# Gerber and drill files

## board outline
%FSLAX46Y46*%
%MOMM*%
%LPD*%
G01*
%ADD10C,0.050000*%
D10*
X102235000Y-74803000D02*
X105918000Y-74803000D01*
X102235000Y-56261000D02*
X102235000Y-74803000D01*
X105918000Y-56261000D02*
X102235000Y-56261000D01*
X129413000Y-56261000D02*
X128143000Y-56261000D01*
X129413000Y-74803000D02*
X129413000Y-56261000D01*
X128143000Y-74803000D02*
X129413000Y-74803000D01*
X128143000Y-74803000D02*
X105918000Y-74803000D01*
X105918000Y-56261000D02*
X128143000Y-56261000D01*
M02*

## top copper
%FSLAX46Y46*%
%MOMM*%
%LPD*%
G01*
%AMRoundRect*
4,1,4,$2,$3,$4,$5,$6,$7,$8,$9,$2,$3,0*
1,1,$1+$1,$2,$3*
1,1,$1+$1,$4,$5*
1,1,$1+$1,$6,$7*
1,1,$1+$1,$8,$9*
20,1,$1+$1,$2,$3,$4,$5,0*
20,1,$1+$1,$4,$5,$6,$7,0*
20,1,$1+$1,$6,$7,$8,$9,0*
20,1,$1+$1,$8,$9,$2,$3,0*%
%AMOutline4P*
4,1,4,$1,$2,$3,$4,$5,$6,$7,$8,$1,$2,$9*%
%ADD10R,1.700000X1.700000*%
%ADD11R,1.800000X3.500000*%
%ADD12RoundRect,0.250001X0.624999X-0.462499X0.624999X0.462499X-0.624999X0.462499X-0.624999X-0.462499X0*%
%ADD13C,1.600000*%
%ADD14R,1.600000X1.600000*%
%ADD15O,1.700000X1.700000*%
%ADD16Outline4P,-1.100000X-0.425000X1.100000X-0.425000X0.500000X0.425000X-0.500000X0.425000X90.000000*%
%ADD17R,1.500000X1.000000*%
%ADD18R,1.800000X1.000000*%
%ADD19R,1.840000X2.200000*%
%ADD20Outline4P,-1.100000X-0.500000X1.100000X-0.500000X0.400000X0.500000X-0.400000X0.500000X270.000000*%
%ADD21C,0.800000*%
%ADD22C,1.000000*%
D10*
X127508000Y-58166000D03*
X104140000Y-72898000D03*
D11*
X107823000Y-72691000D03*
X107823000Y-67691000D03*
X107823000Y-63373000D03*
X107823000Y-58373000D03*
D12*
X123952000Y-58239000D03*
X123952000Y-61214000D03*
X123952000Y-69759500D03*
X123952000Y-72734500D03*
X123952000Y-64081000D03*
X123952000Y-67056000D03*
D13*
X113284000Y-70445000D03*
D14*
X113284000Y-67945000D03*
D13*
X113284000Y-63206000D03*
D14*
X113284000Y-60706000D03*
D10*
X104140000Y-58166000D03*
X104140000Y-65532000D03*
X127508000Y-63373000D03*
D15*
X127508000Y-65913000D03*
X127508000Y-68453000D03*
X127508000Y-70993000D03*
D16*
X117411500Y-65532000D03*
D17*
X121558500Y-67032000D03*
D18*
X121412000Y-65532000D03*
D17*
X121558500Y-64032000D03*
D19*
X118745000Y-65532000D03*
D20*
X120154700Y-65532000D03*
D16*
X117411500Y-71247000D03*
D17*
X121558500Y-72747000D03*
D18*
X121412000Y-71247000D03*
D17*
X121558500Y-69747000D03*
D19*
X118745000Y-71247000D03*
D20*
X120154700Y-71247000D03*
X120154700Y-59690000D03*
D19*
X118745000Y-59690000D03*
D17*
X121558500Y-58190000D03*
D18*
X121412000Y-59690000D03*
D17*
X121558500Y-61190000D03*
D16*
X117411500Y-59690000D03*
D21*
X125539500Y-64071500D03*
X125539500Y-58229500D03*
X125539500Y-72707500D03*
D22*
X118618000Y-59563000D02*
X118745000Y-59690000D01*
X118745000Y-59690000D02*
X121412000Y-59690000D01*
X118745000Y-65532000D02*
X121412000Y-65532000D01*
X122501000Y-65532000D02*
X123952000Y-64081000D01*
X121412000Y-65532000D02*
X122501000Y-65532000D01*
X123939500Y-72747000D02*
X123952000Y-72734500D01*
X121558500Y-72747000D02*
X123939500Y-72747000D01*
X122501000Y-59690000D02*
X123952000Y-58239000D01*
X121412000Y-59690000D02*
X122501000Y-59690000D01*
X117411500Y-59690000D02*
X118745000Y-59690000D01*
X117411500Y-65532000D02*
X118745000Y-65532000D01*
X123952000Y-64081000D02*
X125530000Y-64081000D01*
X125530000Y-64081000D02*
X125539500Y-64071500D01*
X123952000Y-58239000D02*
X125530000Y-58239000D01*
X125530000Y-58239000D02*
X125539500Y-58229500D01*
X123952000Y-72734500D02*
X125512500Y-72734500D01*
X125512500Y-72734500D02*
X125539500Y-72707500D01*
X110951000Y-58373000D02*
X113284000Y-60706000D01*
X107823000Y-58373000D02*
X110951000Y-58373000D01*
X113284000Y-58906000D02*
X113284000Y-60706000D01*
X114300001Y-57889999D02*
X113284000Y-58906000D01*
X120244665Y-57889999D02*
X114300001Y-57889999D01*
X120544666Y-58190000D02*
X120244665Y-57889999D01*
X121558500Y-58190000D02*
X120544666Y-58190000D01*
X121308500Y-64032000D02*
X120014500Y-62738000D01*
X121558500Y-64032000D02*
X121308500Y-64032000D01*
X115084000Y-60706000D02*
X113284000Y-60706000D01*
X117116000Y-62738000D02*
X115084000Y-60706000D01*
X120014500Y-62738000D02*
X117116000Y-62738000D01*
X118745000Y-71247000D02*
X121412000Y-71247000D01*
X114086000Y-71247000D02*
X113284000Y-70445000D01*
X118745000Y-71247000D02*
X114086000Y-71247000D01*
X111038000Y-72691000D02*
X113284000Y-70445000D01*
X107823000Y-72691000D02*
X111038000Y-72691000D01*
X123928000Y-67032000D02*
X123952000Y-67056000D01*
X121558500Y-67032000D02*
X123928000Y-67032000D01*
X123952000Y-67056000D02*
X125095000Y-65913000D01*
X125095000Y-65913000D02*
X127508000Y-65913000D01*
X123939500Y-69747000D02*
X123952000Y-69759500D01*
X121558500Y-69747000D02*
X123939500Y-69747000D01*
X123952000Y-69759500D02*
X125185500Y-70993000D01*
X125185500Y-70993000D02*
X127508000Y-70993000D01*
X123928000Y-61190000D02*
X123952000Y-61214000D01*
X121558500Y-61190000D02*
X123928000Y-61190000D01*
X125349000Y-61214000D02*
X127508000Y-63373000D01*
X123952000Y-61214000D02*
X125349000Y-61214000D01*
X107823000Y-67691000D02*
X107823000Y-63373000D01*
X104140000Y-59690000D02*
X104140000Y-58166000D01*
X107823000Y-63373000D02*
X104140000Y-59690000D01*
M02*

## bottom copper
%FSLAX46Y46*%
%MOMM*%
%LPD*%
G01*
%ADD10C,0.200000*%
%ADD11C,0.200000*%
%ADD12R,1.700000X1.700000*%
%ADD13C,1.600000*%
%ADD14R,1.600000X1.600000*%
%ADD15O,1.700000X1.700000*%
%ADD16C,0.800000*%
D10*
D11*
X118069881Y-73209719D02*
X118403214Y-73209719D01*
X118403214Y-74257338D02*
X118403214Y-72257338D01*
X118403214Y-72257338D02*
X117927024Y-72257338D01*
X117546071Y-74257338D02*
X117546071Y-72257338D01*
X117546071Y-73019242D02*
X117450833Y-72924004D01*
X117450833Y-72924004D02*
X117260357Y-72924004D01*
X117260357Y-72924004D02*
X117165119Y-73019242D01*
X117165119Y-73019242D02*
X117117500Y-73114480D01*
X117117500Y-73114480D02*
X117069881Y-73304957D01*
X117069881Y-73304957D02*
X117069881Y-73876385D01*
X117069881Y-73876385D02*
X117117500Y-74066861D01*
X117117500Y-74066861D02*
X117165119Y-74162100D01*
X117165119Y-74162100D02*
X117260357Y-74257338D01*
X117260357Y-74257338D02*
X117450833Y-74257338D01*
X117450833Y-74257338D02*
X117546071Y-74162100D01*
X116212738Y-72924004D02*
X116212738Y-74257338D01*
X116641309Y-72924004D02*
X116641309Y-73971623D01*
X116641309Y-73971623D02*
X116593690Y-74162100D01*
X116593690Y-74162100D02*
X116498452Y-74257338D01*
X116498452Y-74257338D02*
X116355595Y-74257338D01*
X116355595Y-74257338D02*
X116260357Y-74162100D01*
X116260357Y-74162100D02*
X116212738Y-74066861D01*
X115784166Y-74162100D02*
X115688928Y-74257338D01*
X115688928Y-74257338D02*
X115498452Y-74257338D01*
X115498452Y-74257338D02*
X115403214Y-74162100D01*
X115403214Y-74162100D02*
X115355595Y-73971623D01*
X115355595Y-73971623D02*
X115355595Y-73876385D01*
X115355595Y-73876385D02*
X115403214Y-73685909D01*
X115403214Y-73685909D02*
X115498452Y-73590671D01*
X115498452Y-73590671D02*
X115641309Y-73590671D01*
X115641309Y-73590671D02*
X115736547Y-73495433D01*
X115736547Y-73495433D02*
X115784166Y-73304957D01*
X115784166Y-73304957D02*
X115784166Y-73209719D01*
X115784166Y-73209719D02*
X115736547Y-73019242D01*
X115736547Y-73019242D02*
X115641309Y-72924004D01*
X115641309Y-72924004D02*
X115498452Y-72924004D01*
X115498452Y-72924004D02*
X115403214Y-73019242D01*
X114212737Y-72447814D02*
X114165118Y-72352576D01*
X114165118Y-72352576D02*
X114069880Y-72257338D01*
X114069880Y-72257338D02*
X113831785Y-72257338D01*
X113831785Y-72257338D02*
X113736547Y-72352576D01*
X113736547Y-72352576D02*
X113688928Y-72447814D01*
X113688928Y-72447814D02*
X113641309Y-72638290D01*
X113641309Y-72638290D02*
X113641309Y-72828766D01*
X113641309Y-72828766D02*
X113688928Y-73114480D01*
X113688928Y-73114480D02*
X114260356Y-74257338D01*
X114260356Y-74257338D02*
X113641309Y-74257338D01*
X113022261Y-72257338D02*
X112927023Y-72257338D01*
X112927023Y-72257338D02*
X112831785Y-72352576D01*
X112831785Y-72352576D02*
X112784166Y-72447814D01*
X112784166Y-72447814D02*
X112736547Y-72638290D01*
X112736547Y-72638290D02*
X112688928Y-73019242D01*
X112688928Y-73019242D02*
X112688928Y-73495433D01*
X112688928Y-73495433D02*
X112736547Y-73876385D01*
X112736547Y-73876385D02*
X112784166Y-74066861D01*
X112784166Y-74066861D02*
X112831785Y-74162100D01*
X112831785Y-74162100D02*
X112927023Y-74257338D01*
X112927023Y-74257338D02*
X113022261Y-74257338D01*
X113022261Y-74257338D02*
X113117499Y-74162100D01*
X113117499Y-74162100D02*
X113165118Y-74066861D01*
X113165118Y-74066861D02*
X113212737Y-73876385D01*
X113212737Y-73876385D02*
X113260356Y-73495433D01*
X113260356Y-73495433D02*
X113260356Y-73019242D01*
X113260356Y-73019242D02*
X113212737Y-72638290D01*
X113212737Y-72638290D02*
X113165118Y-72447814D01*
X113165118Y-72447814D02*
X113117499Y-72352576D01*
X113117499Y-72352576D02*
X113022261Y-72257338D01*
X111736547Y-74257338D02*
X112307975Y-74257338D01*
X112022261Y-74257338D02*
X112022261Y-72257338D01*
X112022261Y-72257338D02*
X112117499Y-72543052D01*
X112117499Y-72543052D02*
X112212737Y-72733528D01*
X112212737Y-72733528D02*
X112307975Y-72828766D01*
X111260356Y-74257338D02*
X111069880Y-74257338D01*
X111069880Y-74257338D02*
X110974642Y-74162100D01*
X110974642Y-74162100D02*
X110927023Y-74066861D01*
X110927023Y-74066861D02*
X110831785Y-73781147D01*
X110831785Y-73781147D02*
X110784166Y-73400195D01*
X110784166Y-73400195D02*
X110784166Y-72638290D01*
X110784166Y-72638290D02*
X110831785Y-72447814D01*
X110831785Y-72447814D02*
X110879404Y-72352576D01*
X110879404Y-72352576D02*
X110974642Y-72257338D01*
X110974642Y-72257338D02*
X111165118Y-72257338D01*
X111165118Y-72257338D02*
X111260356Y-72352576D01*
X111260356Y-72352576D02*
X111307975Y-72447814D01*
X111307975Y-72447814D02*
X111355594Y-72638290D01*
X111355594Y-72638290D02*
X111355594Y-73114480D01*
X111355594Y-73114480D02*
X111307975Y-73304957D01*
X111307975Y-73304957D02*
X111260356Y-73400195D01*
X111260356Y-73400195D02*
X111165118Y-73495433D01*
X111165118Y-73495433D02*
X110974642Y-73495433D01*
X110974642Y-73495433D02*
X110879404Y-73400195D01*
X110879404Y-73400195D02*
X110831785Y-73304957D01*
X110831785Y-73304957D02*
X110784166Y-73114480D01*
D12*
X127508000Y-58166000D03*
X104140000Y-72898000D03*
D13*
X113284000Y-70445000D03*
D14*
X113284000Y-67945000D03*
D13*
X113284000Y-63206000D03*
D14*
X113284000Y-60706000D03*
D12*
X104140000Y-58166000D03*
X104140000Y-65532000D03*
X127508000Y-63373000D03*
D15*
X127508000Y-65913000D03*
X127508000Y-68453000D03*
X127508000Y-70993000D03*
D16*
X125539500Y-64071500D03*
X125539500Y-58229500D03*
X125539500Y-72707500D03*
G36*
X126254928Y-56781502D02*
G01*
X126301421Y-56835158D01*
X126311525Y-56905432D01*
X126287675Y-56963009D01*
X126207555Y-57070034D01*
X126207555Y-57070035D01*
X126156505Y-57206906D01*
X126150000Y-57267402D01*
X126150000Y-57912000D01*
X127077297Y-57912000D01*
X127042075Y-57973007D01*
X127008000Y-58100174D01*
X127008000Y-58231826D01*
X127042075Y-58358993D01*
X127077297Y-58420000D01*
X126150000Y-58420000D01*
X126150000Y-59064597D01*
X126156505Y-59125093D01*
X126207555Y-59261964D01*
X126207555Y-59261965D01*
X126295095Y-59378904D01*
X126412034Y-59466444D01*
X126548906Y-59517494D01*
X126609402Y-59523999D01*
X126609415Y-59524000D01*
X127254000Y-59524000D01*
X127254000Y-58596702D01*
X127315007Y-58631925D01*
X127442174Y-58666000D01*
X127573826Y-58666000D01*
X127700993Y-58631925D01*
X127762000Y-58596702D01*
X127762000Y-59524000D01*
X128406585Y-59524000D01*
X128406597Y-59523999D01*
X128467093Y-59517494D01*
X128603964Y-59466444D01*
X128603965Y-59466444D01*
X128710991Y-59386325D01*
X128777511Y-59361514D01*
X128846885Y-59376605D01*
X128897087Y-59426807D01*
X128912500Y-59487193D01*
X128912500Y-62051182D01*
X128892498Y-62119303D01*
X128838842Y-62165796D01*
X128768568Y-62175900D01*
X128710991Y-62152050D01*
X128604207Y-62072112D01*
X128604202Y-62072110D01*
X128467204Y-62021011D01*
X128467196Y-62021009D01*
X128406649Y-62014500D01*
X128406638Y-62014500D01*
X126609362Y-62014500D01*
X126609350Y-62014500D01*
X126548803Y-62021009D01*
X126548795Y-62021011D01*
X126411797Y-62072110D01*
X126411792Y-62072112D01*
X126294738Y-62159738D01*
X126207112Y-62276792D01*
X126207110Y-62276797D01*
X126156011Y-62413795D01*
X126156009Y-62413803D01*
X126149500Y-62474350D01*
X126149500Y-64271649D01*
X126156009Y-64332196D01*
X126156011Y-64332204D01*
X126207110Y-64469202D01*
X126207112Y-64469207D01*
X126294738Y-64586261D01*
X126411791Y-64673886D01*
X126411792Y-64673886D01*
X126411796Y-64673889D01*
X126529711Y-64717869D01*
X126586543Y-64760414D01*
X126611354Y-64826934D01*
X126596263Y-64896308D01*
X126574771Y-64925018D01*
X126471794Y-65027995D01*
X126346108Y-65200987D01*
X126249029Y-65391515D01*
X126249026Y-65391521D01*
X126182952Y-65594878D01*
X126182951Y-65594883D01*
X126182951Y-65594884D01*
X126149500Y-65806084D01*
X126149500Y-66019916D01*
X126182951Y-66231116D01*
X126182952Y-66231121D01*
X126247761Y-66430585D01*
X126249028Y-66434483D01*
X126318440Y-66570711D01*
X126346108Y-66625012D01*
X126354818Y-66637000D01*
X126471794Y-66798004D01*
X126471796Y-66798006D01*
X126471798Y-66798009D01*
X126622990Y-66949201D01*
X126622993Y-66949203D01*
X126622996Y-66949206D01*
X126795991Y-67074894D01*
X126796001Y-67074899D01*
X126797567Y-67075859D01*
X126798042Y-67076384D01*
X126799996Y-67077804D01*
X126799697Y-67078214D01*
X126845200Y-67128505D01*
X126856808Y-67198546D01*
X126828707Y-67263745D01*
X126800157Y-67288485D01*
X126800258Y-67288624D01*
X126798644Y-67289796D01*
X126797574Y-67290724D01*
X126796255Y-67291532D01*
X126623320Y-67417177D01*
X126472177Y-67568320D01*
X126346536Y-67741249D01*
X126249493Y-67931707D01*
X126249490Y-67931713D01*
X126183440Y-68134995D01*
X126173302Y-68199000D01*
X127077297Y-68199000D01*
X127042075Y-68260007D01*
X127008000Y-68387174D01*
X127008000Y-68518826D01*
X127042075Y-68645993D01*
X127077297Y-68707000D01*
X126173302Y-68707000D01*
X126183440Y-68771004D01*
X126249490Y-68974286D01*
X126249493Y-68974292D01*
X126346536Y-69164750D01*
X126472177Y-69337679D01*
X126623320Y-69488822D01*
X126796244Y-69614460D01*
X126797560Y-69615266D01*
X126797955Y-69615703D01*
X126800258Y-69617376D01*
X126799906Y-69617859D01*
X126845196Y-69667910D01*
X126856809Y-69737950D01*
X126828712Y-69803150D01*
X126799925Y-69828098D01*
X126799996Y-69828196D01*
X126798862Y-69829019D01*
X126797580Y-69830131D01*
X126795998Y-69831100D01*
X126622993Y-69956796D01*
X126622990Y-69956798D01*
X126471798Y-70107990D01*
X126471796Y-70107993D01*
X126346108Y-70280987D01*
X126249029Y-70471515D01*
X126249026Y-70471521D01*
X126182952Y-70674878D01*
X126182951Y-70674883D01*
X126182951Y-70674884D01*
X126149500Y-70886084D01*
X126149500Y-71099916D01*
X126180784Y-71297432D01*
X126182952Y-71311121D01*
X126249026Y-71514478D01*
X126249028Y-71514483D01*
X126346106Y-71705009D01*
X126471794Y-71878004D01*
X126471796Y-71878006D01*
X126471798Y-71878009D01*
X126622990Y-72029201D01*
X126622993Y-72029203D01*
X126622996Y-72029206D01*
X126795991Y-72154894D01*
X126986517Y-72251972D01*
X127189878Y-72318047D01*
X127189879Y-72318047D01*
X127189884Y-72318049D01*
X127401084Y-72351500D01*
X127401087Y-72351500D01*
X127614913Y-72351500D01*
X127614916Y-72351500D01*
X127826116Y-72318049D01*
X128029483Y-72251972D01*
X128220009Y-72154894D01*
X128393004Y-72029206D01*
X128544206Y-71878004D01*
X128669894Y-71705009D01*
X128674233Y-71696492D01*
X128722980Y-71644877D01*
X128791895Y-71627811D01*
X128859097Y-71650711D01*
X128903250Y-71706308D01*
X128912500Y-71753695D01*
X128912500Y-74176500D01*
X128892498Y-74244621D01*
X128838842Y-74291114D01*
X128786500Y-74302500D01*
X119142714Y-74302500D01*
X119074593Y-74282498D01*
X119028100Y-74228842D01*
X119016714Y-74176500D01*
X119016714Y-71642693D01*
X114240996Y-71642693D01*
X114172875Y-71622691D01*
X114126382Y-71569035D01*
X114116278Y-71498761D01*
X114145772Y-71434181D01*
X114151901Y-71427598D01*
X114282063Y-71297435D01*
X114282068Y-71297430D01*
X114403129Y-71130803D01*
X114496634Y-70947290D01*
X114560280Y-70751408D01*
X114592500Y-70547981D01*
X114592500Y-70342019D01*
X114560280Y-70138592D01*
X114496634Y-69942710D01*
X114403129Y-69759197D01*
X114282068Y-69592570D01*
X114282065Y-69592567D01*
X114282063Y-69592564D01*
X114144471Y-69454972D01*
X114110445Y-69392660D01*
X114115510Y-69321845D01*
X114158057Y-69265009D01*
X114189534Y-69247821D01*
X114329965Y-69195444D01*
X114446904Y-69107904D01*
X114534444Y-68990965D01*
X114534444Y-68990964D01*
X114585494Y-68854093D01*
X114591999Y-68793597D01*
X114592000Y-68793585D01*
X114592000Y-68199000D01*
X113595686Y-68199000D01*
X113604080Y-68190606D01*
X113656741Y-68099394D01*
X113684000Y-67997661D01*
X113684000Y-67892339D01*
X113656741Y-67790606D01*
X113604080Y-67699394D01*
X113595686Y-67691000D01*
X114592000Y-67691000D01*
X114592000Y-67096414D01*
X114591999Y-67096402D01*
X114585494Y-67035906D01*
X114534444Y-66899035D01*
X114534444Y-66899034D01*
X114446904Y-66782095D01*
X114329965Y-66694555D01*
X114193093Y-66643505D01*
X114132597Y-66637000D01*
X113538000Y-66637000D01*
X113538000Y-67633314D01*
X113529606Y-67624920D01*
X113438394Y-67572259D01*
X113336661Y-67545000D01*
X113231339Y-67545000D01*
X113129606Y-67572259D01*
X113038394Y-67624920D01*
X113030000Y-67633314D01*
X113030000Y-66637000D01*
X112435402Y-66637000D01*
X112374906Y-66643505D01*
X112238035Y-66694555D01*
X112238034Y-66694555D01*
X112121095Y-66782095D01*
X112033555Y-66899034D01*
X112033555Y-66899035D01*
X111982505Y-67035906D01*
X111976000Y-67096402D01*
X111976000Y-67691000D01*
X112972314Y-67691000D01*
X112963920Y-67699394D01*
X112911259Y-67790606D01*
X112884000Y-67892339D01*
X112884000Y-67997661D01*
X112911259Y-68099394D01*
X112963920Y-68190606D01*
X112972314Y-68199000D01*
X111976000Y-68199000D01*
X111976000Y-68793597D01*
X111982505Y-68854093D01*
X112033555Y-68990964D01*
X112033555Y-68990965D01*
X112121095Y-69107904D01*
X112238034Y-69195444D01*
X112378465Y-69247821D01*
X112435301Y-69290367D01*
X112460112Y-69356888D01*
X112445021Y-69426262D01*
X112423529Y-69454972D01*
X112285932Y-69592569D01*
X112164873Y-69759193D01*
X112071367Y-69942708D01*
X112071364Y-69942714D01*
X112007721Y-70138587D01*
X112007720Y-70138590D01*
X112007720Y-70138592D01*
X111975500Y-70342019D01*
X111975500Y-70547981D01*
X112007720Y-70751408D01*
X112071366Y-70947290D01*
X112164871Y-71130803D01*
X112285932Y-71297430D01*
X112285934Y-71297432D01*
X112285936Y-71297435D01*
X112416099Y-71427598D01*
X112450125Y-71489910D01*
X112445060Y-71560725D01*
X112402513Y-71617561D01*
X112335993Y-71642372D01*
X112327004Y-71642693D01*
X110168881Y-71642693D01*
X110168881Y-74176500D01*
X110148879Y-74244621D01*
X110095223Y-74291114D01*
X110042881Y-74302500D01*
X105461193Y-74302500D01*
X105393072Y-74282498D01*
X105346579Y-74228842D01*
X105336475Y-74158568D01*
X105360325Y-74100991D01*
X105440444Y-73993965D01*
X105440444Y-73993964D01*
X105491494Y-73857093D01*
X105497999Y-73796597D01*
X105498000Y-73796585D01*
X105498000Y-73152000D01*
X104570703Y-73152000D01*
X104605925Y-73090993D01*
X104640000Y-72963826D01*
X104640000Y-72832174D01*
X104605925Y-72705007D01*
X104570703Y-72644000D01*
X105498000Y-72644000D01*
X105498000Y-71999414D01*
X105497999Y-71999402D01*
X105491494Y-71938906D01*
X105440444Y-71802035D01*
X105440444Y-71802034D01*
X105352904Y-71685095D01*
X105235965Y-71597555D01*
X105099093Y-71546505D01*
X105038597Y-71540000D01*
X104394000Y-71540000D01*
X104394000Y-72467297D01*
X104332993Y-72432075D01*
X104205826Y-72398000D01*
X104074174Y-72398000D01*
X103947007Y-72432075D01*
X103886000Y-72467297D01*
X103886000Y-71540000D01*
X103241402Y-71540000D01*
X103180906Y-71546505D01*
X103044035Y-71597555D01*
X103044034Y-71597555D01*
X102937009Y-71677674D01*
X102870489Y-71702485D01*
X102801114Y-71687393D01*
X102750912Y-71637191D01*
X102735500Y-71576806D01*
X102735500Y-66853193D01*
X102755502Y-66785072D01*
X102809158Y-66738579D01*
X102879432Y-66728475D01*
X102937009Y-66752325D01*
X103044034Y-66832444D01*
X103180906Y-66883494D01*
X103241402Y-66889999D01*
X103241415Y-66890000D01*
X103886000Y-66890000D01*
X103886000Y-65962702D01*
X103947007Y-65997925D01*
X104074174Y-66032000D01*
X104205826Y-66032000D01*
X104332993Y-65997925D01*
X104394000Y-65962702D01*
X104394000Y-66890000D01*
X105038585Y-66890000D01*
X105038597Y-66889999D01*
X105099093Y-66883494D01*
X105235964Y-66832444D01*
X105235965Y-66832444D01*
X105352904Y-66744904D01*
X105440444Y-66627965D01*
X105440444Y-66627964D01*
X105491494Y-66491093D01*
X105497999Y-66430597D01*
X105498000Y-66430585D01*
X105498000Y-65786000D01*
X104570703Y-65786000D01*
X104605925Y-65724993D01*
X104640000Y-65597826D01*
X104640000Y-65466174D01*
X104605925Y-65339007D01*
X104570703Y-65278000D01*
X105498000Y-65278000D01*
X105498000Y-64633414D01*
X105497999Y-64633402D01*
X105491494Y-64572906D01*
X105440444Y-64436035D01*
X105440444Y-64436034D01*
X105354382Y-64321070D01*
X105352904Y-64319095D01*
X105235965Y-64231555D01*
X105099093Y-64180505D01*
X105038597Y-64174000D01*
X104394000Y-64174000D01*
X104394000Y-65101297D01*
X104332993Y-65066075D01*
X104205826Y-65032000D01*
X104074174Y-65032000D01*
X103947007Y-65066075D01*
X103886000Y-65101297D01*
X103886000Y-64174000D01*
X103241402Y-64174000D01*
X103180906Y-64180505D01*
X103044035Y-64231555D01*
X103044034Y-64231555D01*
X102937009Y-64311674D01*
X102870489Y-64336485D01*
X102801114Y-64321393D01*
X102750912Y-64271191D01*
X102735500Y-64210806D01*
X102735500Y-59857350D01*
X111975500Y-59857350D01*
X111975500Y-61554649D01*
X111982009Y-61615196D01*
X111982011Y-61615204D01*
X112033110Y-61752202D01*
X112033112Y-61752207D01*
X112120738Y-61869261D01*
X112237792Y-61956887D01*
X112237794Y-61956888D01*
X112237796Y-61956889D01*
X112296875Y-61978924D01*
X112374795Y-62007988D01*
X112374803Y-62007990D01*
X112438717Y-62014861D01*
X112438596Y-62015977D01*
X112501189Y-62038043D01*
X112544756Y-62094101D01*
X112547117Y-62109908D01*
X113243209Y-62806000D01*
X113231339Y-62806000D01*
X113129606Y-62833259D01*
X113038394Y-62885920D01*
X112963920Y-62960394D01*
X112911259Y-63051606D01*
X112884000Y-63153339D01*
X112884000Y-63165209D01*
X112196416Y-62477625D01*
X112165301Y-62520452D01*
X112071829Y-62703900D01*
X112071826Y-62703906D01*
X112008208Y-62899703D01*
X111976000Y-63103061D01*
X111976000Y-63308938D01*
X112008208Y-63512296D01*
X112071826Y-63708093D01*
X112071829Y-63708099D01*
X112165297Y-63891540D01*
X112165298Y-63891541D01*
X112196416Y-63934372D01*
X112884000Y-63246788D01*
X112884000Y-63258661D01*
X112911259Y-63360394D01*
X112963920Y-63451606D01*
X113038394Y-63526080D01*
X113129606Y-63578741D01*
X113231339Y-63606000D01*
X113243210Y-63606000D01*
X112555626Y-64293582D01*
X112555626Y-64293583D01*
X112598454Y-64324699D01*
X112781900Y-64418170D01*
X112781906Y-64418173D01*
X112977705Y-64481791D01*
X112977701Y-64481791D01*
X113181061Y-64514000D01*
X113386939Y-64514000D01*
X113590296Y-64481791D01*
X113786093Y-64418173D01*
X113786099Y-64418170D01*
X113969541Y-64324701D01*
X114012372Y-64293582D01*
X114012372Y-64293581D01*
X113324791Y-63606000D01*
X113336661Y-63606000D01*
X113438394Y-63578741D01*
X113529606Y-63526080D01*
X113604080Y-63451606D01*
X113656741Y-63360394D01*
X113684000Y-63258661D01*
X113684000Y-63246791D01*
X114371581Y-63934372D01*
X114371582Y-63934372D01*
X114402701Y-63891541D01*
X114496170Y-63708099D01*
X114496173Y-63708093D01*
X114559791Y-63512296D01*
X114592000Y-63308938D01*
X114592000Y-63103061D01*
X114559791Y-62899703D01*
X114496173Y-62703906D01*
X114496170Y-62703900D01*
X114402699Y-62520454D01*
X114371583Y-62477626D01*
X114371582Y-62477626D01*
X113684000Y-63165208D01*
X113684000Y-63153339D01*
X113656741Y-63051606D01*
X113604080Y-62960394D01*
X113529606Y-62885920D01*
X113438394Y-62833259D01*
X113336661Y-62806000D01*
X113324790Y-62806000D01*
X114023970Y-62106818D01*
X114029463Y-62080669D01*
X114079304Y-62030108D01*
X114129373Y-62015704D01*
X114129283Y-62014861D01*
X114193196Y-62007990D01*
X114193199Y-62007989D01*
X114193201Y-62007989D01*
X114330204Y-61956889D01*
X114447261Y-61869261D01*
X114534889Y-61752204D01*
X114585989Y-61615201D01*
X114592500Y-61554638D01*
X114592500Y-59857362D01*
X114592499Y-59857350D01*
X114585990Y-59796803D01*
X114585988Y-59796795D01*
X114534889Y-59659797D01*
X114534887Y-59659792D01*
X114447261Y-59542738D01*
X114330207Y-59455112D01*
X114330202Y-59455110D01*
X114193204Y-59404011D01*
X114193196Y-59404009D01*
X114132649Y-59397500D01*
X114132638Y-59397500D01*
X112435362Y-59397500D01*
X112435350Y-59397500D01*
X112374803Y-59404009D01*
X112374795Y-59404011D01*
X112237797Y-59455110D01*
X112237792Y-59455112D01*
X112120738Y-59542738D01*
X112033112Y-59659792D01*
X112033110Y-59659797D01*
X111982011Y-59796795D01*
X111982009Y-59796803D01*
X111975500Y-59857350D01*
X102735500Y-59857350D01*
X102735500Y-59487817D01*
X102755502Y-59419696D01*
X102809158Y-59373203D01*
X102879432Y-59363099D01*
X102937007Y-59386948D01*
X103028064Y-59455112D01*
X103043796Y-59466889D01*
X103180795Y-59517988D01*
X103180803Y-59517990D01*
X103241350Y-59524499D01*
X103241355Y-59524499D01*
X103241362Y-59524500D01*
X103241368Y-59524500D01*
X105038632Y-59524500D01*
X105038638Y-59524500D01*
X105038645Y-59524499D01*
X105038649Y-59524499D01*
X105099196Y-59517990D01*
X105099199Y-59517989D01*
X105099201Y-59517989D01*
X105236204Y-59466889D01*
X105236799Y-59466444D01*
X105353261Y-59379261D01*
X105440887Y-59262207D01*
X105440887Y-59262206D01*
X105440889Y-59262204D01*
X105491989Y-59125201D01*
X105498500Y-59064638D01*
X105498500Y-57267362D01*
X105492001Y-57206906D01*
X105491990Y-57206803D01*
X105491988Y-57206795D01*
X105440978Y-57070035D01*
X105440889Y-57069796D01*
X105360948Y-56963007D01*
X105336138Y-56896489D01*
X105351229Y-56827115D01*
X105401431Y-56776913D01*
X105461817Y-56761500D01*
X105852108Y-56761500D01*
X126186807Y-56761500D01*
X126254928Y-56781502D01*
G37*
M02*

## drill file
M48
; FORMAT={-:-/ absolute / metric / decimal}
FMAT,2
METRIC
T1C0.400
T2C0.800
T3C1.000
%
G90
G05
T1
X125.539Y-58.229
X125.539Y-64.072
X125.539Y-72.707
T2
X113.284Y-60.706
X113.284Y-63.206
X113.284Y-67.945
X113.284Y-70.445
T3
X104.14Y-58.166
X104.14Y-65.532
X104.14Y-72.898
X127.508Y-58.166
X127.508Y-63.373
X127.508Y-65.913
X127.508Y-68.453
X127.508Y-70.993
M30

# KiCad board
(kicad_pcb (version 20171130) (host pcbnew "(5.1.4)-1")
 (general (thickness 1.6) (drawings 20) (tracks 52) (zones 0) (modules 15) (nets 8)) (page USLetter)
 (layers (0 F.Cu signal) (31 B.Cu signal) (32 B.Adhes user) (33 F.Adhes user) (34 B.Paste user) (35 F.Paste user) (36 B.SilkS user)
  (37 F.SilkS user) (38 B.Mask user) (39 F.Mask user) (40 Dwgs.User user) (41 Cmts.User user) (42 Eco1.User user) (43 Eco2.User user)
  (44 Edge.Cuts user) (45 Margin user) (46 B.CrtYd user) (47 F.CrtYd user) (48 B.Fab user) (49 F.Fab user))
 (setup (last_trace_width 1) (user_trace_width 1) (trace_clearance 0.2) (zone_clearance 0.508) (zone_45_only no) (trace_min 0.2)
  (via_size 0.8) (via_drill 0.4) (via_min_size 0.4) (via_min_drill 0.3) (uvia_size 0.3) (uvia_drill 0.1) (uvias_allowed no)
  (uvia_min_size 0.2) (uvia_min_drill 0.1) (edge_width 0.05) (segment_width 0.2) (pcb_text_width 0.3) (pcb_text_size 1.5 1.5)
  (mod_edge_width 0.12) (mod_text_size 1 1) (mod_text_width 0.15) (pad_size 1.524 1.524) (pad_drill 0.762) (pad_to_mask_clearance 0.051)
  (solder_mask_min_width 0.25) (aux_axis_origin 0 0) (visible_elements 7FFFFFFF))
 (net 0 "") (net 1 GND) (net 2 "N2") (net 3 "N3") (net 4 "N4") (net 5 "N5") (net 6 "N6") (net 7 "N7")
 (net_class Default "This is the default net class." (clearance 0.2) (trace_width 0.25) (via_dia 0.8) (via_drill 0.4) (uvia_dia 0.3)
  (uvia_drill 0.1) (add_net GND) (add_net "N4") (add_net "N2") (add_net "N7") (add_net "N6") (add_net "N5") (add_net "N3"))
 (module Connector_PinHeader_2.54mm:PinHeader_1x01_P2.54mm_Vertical (layer F.Cu) (at 127.508 58.166)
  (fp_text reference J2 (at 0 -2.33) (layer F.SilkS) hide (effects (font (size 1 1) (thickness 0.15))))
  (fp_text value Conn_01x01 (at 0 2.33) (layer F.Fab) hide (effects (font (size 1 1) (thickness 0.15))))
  (pad 1 thru_hole rect (at 0 0) (size 1.7 1.7) (drill 1) (layers *.Cu *.Mask) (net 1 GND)))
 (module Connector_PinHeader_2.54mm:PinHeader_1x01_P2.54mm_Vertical (layer F.Cu) (at 104.14 72.898)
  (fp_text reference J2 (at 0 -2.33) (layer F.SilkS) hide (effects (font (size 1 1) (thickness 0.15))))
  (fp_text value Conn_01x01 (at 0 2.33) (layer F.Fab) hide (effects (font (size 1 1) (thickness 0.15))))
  (pad 1 thru_hole rect (at 0 0) (size 1.7 1.7) (drill 1) (layers *.Cu *.Mask) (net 1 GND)))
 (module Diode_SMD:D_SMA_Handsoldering (layer F.Cu) (at 107.823 70.191 270)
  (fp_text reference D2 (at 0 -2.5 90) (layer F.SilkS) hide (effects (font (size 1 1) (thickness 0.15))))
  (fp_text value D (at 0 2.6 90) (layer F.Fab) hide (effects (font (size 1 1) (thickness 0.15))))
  (pad 2 smd rect (at 2.5 0 270) (size 3.5 1.8) (layers F.Cu F.Paste F.Mask) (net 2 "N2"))
  (pad 1 smd rect (at -2.5 0 270) (size 3.5 1.8) (layers F.Cu F.Paste F.Mask) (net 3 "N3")))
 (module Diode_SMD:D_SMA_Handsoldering (layer F.Cu) (at 107.823 60.873 270)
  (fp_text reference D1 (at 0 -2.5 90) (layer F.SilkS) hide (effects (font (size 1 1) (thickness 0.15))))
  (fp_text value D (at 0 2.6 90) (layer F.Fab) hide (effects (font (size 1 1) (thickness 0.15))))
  (pad 2 smd rect (at 2.5 0 270) (size 3.5 1.8) (layers F.Cu F.Paste F.Mask) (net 3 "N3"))
  (pad 1 smd rect (at -2.5 0 270) (size 3.5 1.8) (layers F.Cu F.Paste F.Mask) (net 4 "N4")))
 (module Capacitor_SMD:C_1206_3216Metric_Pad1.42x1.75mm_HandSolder (layer F.Cu) (at 123.952 59.7265 90)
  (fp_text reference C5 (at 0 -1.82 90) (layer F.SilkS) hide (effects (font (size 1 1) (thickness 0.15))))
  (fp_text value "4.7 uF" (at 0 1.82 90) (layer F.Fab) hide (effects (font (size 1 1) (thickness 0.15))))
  (pad 2 smd roundrect (at 1.4875 0 90) (size 1.425 1.75) (layers F.Cu F.Paste F.Mask) (roundrect_rratio 0.175439) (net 1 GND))
  (pad 1 smd roundrect (at -1.4875 0 90) (size 1.425 1.75) (layers F.Cu F.Paste F.Mask) (roundrect_rratio 0.175439) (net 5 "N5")))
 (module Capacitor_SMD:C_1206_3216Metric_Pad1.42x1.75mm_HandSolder (layer F.Cu) (at 123.952 71.247 90)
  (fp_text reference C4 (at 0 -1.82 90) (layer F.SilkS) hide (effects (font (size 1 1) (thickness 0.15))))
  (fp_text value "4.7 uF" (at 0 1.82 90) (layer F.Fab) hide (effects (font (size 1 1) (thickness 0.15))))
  (pad 2 smd roundrect (at 1.4875 0 90) (size 1.425 1.75) (layers F.Cu F.Paste F.Mask) (roundrect_rratio 0.175439) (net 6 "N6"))
  (pad 1 smd roundrect (at -1.4875 0 90) (size 1.425 1.75) (layers F.Cu F.Paste F.Mask) (roundrect_rratio 0.175439) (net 1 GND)))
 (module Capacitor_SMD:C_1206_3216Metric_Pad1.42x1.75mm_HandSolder (layer F.Cu) (at 123.952 65.5685 90)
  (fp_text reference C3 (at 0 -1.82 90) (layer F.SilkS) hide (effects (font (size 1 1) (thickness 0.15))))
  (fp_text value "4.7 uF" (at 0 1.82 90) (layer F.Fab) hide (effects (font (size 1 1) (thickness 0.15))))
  (pad 2 smd roundrect (at 1.4875 0 90) (size 1.425 1.75) (layers F.Cu F.Paste F.Mask) (roundrect_rratio 0.175439) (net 1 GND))
  (pad 1 smd roundrect (at -1.4875 0 90) (size 1.425 1.75) (layers F.Cu F.Paste F.Mask) (roundrect_rratio 0.175439) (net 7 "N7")))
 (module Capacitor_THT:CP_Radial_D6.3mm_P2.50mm (layer F.Cu) (at 113.284 67.945 270)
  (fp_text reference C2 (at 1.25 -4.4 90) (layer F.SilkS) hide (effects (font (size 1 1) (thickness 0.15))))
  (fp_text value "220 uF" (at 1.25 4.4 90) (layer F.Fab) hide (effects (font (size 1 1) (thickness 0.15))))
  (pad 2 thru_hole circle (at 2.5 0 270) (size 1.6 1.6) (drill 0.8) (layers *.Cu *.Mask) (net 2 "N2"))
  (pad 1 thru_hole rect (at 0 0 270) (size 1.6 1.6) (drill 0.8) (layers *.Cu *.Mask) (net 1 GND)))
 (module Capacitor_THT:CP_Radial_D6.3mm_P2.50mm (layer F.Cu) (at 113.284 60.706 270)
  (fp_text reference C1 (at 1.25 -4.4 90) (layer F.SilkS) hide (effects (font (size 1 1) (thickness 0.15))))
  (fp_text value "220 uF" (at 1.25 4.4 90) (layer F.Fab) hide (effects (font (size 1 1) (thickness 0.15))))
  (pad 2 thru_hole circle (at 2.5 0 270) (size 1.6 1.6) (drill 0.8) (layers *.Cu *.Mask) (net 1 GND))
  (pad 1 thru_hole rect (at 0 0 270) (size 1.6 1.6) (drill 0.8) (layers *.Cu *.Mask) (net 4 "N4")))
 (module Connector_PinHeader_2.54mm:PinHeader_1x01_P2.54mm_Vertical (layer F.Cu) (at 104.14 58.166)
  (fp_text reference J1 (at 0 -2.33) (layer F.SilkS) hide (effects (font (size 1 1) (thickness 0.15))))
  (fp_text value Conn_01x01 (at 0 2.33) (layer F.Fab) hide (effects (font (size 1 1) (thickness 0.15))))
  (pad 1 thru_hole rect (at 0 0) (size 1.7 1.7) (drill 1) (layers *.Cu *.Mask) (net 3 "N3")))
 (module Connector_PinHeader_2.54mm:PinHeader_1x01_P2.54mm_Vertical (layer F.Cu) (at 104.14 65.532)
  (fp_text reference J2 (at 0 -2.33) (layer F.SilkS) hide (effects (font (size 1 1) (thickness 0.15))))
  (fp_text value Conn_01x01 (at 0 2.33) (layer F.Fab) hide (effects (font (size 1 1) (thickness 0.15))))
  (pad 1 thru_hole rect (at 0 0) (size 1.7 1.7) (drill 1) (layers *.Cu *.Mask) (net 1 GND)))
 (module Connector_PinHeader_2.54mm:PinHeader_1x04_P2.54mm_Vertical (layer F.Cu) (at 127.508 63.373)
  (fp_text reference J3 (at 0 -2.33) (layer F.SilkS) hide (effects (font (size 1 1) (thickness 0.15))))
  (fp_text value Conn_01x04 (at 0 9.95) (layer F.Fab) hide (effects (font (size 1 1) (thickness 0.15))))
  (pad 1 thru_hole rect (at 0 0) (size 1.7 1.7) (drill 1) (layers *.Cu *.Mask) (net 5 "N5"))
  (pad 2 thru_hole oval (at 0 2.54) (size 1.7 1.7) (drill 1) (layers *.Cu *.Mask) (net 7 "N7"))
  (pad 3 thru_hole oval (at 0 5.08) (size 1.7 1.7) (drill 1) (layers *.Cu *.Mask) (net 1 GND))
  (pad 4 thru_hole oval (at 0 7.62) (size 1.7 1.7) (drill 1) (layers *.Cu *.Mask) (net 6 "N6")))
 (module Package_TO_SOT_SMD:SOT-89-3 (layer F.Cu) (at 120.0785 65.532 180)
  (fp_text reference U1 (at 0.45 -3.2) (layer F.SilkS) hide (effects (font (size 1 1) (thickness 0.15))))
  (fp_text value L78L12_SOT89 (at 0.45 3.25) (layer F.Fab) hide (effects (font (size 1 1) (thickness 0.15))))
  (pad 2 smd trapezoid (at 2.667 0 90) (size 1.6 0.85) (rect_delta 0 0.6) (layers F.Cu F.Paste F.Mask) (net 1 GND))
  (pad 1 smd rect (at -1.48 -1.5 90) (size 1 1.5) (layers F.Cu F.Paste F.Mask) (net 7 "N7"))
  (pad 2 smd rect (at -1.3335 0 90) (size 1 1.8) (layers F.Cu F.Paste F.Mask) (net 1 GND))
  (pad 3 smd rect (at -1.48 1.5 90) (size 1 1.5) (layers F.Cu F.Paste F.Mask) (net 4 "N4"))
  (pad 2 smd rect (at 1.3335 0 90) (size 2.2 1.84) (layers F.Cu F.Paste F.Mask) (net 1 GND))
  (pad 2 smd trapezoid (at -0.0762 0 270) (size 1.5 1) (rect_delta 0 0.7) (layers F.Cu F.Paste F.Mask) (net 1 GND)))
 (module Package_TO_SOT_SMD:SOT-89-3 (layer F.Cu) (at 120.0785 71.247 180)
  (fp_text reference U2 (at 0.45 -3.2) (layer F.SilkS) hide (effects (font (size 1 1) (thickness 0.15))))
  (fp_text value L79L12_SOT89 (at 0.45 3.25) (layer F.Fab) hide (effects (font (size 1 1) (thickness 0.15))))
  (pad 2 smd trapezoid (at 2.667 0 90) (size 1.6 0.85) (rect_delta 0 0.6) (layers F.Cu F.Paste F.Mask) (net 2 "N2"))
  (pad 1 smd rect (at -1.48 -1.5 90) (size 1 1.5) (layers F.Cu F.Paste F.Mask) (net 1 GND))
  (pad 2 smd rect (at -1.3335 0 90) (size 1 1.8) (layers F.Cu F.Paste F.Mask) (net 2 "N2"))
  (pad 3 smd rect (at -1.48 1.5 90) (size 1 1.5) (layers F.Cu F.Paste F.Mask) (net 6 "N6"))
  (pad 2 smd rect (at 1.3335 0 90) (size 2.2 1.84) (layers F.Cu F.Paste F.Mask) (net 2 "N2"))
  (pad 2 smd trapezoid (at -0.0762 0 270) (size 1.5 1) (rect_delta 0 0.7) (layers F.Cu F.Paste F.Mask) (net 2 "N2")))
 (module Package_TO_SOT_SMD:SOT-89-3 (layer F.Cu) (at 120.0785 59.69 180)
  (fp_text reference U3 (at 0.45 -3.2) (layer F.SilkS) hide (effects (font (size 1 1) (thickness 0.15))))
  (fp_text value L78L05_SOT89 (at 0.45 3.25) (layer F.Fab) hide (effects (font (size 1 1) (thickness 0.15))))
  (pad 2 smd trapezoid (at -0.0762 0 270) (size 1.5 1) (rect_delta 0 0.7) (layers F.Cu F.Paste F.Mask) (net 1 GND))
  (pad 2 smd rect (at 1.3335 0 90) (size 2.2 1.84) (layers F.Cu F.Paste F.Mask) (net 1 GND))
  (pad 3 smd rect (at -1.48 1.5 90) (size 1 1.5) (layers F.Cu F.Paste F.Mask) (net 4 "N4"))
  (pad 2 smd rect (at -1.3335 0 90) (size 1 1.8) (layers F.Cu F.Paste F.Mask) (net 1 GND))
  (pad 1 smd rect (at -1.48 -1.5 90) (size 1 1.5) (layers F.Cu F.Paste F.Mask) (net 5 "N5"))
  (pad 2 smd trapezoid (at 2.667 0 90) (size 1.6 0.85) (rect_delta 0 0.6) (layers F.Cu F.Paste F.Mask) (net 1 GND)))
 (gr_line (start 102.235 74.803) (end 105.918 74.803) (layer Edge.Cuts) (width 0.05))
 (gr_line (start 102.235 56.261) (end 102.235 74.803) (layer Edge.Cuts) (width 0.05))
 (gr_line (start 105.918 56.261) (end 102.235 56.261) (layer Edge.Cuts) (width 0.05))
 (gr_line (start 129.413 56.261) (end 128.143 56.261) (layer Edge.Cuts) (width 0.05))
 (gr_line (start 129.413 74.803) (end 129.413 56.261) (layer Edge.Cuts) (width 0.05))
 (gr_line (start 128.143 74.803) (end 129.413 74.803) (layer Edge.Cuts) (width 0.05))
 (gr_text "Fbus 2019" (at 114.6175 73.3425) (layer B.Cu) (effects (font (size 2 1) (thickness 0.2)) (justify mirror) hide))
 (gr_line (start 128.143 74.803) (end 105.918 74.803) (layer Edge.Cuts) (width 0.05))
 (gr_line (start 105.918 56.261) (end 128.143 56.261) (layer Edge.Cuts) (width 0.05))
 (segment (start 118.618 59.563) (end 118.745 59.69) (width 1) (layer F.Cu) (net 1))
 (segment (start 118.745 59.69) (end 121.412 59.69) (width 1) (layer F.Cu) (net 1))
 (segment (start 118.745 65.532) (end 121.412 65.532) (width 1) (layer F.Cu) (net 1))
 (segment (start 122.501 65.532) (end 123.952 64.081) (width 1) (layer F.Cu) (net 1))
 (segment (start 121.412 65.532) (end 122.501 65.532) (width 1) (layer F.Cu) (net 1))
 (segment (start 123.9395 72.747) (end 123.952 72.7345) (width 1) (layer F.Cu) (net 1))
 (segment (start 121.5585 72.747) (end 123.9395 72.747) (width 1) (layer F.Cu) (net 1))
 (segment (start 122.501 59.69) (end 123.952 58.239) (width 1) (layer F.Cu) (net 1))
 (segment (start 121.412 59.69) (end 122.501 59.69) (width 1) (layer F.Cu) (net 1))
 (segment (start 117.4115 59.69) (end 118.745 59.69) (width 1) (layer F.Cu) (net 1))
 (segment (start 117.4115 65.532) (end 118.745 65.532) (width 1) (layer F.Cu) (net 1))
 (via (at 125.5395 64.0715) (size 0.8) (drill 0.4) (layers F.Cu B.Cu) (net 1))
 (segment (start 123.952 64.081) (end 125.53 64.081) (width 1) (layer F.Cu) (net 1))
 (segment (start 125.53 64.081) (end 125.5395 64.0715) (width 1) (layer F.Cu) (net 1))
 (via (at 125.5395 58.2295) (size 0.8) (drill 0.4) (layers F.Cu B.Cu) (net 1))
 (segment (start 123.952 58.239) (end 125.53 58.239) (width 1) (layer F.Cu) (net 1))
 (segment (start 125.53 58.239) (end 125.5395 58.2295) (width 1) (layer F.Cu) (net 1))
 (via (at 125.5395 72.7075) (size 0.8) (drill 0.4) (layers F.Cu B.Cu) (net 1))
 (segment (start 123.952 72.7345) (end 125.5125 72.7345) (width 1) (layer F.Cu) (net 1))
 (segment (start 125.5125 72.7345) (end 125.5395 72.7075) (width 1) (layer F.Cu) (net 1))
 (segment (start 110.951 58.373) (end 113.284 60.706) (width 1) (layer F.Cu) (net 4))
 (segment (start 107.823 58.373) (end 110.951 58.373) (width 1) (layer F.Cu) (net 4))
 (segment (start 113.284 58.906) (end 113.284 60.706) (width 1) (layer F.Cu) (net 4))
 (segment (start 114.300001 57.889999) (end 113.284 58.906) (width 1) (layer F.Cu) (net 4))
 (segment (start 120.244665 57.889999) (end 114.300001 57.889999) (width 1) (layer F.Cu) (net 4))
 (segment (start 120.544666 58.19) (end 120.244665 57.889999) (width 1) (layer F.Cu) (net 4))
 (segment (start 121.5585 58.19) (end 120.544666 58.19) (width 1) (layer F.Cu) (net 4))
 (segment (start 121.3085 64.032) (end 120.0145 62.738) (width 1) (layer F.Cu) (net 4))
 (segment (start 121.5585 64.032) (end 121.3085 64.032) (width 1) (layer F.Cu) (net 4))
 (segment (start 115.084 60.706) (end 113.284 60.706) (width 1) (layer F.Cu) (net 4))
 (segment (start 117.116 62.738) (end 115.084 60.706) (width 1) (layer F.Cu) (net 4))
 (segment (start 120.0145 62.738) (end 117.116 62.738) (width 1) (layer F.Cu) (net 4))
 (segment (start 118.745 71.247) (end 121.412 71.247) (width 1) (layer F.Cu) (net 2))
 (segment (start 114.086 71.247) (end 113.284 70.445) (width 1) (layer F.Cu) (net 2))
 (segment (start 118.745 71.247) (end 114.086 71.247) (width 1) (layer F.Cu) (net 2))
 (segment (start 111.038 72.691) (end 113.284 70.445) (width 1) (layer F.Cu) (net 2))
 (segment (start 107.823 72.691) (end 111.038 72.691) (width 1) (layer F.Cu) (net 2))
 (segment (start 123.928 67.032) (end 123.952 67.056) (width 1) (layer F.Cu) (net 7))
 (segment (start 121.5585 67.032) (end 123.928 67.032) (width 1) (layer F.Cu) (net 7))
 (segment (start 123.952 67.056) (end 125.095 65.913) (width 1) (layer F.Cu) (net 7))
 (segment (start 125.095 65.913) (end 127.508 65.913) (width 1) (layer F.Cu) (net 7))
 (segment (start 123.9395 69.747) (end 123.952 69.7595) (width 1) (layer F.Cu) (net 6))
 (segment (start 121.5585 69.747) (end 123.9395 69.747) (width 1) (layer F.Cu) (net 6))
 (segment (start 123.952 69.7595) (end 125.1855 70.993) (width 1) (layer F.Cu) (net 6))
 (segment (start 125.1855 70.993) (end 127.508 70.993) (width 1) (layer F.Cu) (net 6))
 (segment (start 123.928 61.19) (end 123.952 61.214) (width 1) (layer F.Cu) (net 5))
 (segment (start 121.5585 61.19) (end 123.928 61.19) (width 1) (layer F.Cu) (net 5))
 (segment (start 125.349 61.214) (end 127.508 63.373) (width 1) (layer F.Cu) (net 5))
 (segment (start 123.952 61.214) (end 125.349 61.214) (width 1) (layer F.Cu) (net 5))
 (segment (start 107.823 67.691) (end 107.823 63.373) (width 1) (layer F.Cu) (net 3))
 (segment (start 104.14 59.69) (end 104.14 58.166) (width 1) (layer F.Cu) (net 3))
 (segment (start 107.823 63.373) (end 104.14 59.69) (width 1) (layer F.Cu) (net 3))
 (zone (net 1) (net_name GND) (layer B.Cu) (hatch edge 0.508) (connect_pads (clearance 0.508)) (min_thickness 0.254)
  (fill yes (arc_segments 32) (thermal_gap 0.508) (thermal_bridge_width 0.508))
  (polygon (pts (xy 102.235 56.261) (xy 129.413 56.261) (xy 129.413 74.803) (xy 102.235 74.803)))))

